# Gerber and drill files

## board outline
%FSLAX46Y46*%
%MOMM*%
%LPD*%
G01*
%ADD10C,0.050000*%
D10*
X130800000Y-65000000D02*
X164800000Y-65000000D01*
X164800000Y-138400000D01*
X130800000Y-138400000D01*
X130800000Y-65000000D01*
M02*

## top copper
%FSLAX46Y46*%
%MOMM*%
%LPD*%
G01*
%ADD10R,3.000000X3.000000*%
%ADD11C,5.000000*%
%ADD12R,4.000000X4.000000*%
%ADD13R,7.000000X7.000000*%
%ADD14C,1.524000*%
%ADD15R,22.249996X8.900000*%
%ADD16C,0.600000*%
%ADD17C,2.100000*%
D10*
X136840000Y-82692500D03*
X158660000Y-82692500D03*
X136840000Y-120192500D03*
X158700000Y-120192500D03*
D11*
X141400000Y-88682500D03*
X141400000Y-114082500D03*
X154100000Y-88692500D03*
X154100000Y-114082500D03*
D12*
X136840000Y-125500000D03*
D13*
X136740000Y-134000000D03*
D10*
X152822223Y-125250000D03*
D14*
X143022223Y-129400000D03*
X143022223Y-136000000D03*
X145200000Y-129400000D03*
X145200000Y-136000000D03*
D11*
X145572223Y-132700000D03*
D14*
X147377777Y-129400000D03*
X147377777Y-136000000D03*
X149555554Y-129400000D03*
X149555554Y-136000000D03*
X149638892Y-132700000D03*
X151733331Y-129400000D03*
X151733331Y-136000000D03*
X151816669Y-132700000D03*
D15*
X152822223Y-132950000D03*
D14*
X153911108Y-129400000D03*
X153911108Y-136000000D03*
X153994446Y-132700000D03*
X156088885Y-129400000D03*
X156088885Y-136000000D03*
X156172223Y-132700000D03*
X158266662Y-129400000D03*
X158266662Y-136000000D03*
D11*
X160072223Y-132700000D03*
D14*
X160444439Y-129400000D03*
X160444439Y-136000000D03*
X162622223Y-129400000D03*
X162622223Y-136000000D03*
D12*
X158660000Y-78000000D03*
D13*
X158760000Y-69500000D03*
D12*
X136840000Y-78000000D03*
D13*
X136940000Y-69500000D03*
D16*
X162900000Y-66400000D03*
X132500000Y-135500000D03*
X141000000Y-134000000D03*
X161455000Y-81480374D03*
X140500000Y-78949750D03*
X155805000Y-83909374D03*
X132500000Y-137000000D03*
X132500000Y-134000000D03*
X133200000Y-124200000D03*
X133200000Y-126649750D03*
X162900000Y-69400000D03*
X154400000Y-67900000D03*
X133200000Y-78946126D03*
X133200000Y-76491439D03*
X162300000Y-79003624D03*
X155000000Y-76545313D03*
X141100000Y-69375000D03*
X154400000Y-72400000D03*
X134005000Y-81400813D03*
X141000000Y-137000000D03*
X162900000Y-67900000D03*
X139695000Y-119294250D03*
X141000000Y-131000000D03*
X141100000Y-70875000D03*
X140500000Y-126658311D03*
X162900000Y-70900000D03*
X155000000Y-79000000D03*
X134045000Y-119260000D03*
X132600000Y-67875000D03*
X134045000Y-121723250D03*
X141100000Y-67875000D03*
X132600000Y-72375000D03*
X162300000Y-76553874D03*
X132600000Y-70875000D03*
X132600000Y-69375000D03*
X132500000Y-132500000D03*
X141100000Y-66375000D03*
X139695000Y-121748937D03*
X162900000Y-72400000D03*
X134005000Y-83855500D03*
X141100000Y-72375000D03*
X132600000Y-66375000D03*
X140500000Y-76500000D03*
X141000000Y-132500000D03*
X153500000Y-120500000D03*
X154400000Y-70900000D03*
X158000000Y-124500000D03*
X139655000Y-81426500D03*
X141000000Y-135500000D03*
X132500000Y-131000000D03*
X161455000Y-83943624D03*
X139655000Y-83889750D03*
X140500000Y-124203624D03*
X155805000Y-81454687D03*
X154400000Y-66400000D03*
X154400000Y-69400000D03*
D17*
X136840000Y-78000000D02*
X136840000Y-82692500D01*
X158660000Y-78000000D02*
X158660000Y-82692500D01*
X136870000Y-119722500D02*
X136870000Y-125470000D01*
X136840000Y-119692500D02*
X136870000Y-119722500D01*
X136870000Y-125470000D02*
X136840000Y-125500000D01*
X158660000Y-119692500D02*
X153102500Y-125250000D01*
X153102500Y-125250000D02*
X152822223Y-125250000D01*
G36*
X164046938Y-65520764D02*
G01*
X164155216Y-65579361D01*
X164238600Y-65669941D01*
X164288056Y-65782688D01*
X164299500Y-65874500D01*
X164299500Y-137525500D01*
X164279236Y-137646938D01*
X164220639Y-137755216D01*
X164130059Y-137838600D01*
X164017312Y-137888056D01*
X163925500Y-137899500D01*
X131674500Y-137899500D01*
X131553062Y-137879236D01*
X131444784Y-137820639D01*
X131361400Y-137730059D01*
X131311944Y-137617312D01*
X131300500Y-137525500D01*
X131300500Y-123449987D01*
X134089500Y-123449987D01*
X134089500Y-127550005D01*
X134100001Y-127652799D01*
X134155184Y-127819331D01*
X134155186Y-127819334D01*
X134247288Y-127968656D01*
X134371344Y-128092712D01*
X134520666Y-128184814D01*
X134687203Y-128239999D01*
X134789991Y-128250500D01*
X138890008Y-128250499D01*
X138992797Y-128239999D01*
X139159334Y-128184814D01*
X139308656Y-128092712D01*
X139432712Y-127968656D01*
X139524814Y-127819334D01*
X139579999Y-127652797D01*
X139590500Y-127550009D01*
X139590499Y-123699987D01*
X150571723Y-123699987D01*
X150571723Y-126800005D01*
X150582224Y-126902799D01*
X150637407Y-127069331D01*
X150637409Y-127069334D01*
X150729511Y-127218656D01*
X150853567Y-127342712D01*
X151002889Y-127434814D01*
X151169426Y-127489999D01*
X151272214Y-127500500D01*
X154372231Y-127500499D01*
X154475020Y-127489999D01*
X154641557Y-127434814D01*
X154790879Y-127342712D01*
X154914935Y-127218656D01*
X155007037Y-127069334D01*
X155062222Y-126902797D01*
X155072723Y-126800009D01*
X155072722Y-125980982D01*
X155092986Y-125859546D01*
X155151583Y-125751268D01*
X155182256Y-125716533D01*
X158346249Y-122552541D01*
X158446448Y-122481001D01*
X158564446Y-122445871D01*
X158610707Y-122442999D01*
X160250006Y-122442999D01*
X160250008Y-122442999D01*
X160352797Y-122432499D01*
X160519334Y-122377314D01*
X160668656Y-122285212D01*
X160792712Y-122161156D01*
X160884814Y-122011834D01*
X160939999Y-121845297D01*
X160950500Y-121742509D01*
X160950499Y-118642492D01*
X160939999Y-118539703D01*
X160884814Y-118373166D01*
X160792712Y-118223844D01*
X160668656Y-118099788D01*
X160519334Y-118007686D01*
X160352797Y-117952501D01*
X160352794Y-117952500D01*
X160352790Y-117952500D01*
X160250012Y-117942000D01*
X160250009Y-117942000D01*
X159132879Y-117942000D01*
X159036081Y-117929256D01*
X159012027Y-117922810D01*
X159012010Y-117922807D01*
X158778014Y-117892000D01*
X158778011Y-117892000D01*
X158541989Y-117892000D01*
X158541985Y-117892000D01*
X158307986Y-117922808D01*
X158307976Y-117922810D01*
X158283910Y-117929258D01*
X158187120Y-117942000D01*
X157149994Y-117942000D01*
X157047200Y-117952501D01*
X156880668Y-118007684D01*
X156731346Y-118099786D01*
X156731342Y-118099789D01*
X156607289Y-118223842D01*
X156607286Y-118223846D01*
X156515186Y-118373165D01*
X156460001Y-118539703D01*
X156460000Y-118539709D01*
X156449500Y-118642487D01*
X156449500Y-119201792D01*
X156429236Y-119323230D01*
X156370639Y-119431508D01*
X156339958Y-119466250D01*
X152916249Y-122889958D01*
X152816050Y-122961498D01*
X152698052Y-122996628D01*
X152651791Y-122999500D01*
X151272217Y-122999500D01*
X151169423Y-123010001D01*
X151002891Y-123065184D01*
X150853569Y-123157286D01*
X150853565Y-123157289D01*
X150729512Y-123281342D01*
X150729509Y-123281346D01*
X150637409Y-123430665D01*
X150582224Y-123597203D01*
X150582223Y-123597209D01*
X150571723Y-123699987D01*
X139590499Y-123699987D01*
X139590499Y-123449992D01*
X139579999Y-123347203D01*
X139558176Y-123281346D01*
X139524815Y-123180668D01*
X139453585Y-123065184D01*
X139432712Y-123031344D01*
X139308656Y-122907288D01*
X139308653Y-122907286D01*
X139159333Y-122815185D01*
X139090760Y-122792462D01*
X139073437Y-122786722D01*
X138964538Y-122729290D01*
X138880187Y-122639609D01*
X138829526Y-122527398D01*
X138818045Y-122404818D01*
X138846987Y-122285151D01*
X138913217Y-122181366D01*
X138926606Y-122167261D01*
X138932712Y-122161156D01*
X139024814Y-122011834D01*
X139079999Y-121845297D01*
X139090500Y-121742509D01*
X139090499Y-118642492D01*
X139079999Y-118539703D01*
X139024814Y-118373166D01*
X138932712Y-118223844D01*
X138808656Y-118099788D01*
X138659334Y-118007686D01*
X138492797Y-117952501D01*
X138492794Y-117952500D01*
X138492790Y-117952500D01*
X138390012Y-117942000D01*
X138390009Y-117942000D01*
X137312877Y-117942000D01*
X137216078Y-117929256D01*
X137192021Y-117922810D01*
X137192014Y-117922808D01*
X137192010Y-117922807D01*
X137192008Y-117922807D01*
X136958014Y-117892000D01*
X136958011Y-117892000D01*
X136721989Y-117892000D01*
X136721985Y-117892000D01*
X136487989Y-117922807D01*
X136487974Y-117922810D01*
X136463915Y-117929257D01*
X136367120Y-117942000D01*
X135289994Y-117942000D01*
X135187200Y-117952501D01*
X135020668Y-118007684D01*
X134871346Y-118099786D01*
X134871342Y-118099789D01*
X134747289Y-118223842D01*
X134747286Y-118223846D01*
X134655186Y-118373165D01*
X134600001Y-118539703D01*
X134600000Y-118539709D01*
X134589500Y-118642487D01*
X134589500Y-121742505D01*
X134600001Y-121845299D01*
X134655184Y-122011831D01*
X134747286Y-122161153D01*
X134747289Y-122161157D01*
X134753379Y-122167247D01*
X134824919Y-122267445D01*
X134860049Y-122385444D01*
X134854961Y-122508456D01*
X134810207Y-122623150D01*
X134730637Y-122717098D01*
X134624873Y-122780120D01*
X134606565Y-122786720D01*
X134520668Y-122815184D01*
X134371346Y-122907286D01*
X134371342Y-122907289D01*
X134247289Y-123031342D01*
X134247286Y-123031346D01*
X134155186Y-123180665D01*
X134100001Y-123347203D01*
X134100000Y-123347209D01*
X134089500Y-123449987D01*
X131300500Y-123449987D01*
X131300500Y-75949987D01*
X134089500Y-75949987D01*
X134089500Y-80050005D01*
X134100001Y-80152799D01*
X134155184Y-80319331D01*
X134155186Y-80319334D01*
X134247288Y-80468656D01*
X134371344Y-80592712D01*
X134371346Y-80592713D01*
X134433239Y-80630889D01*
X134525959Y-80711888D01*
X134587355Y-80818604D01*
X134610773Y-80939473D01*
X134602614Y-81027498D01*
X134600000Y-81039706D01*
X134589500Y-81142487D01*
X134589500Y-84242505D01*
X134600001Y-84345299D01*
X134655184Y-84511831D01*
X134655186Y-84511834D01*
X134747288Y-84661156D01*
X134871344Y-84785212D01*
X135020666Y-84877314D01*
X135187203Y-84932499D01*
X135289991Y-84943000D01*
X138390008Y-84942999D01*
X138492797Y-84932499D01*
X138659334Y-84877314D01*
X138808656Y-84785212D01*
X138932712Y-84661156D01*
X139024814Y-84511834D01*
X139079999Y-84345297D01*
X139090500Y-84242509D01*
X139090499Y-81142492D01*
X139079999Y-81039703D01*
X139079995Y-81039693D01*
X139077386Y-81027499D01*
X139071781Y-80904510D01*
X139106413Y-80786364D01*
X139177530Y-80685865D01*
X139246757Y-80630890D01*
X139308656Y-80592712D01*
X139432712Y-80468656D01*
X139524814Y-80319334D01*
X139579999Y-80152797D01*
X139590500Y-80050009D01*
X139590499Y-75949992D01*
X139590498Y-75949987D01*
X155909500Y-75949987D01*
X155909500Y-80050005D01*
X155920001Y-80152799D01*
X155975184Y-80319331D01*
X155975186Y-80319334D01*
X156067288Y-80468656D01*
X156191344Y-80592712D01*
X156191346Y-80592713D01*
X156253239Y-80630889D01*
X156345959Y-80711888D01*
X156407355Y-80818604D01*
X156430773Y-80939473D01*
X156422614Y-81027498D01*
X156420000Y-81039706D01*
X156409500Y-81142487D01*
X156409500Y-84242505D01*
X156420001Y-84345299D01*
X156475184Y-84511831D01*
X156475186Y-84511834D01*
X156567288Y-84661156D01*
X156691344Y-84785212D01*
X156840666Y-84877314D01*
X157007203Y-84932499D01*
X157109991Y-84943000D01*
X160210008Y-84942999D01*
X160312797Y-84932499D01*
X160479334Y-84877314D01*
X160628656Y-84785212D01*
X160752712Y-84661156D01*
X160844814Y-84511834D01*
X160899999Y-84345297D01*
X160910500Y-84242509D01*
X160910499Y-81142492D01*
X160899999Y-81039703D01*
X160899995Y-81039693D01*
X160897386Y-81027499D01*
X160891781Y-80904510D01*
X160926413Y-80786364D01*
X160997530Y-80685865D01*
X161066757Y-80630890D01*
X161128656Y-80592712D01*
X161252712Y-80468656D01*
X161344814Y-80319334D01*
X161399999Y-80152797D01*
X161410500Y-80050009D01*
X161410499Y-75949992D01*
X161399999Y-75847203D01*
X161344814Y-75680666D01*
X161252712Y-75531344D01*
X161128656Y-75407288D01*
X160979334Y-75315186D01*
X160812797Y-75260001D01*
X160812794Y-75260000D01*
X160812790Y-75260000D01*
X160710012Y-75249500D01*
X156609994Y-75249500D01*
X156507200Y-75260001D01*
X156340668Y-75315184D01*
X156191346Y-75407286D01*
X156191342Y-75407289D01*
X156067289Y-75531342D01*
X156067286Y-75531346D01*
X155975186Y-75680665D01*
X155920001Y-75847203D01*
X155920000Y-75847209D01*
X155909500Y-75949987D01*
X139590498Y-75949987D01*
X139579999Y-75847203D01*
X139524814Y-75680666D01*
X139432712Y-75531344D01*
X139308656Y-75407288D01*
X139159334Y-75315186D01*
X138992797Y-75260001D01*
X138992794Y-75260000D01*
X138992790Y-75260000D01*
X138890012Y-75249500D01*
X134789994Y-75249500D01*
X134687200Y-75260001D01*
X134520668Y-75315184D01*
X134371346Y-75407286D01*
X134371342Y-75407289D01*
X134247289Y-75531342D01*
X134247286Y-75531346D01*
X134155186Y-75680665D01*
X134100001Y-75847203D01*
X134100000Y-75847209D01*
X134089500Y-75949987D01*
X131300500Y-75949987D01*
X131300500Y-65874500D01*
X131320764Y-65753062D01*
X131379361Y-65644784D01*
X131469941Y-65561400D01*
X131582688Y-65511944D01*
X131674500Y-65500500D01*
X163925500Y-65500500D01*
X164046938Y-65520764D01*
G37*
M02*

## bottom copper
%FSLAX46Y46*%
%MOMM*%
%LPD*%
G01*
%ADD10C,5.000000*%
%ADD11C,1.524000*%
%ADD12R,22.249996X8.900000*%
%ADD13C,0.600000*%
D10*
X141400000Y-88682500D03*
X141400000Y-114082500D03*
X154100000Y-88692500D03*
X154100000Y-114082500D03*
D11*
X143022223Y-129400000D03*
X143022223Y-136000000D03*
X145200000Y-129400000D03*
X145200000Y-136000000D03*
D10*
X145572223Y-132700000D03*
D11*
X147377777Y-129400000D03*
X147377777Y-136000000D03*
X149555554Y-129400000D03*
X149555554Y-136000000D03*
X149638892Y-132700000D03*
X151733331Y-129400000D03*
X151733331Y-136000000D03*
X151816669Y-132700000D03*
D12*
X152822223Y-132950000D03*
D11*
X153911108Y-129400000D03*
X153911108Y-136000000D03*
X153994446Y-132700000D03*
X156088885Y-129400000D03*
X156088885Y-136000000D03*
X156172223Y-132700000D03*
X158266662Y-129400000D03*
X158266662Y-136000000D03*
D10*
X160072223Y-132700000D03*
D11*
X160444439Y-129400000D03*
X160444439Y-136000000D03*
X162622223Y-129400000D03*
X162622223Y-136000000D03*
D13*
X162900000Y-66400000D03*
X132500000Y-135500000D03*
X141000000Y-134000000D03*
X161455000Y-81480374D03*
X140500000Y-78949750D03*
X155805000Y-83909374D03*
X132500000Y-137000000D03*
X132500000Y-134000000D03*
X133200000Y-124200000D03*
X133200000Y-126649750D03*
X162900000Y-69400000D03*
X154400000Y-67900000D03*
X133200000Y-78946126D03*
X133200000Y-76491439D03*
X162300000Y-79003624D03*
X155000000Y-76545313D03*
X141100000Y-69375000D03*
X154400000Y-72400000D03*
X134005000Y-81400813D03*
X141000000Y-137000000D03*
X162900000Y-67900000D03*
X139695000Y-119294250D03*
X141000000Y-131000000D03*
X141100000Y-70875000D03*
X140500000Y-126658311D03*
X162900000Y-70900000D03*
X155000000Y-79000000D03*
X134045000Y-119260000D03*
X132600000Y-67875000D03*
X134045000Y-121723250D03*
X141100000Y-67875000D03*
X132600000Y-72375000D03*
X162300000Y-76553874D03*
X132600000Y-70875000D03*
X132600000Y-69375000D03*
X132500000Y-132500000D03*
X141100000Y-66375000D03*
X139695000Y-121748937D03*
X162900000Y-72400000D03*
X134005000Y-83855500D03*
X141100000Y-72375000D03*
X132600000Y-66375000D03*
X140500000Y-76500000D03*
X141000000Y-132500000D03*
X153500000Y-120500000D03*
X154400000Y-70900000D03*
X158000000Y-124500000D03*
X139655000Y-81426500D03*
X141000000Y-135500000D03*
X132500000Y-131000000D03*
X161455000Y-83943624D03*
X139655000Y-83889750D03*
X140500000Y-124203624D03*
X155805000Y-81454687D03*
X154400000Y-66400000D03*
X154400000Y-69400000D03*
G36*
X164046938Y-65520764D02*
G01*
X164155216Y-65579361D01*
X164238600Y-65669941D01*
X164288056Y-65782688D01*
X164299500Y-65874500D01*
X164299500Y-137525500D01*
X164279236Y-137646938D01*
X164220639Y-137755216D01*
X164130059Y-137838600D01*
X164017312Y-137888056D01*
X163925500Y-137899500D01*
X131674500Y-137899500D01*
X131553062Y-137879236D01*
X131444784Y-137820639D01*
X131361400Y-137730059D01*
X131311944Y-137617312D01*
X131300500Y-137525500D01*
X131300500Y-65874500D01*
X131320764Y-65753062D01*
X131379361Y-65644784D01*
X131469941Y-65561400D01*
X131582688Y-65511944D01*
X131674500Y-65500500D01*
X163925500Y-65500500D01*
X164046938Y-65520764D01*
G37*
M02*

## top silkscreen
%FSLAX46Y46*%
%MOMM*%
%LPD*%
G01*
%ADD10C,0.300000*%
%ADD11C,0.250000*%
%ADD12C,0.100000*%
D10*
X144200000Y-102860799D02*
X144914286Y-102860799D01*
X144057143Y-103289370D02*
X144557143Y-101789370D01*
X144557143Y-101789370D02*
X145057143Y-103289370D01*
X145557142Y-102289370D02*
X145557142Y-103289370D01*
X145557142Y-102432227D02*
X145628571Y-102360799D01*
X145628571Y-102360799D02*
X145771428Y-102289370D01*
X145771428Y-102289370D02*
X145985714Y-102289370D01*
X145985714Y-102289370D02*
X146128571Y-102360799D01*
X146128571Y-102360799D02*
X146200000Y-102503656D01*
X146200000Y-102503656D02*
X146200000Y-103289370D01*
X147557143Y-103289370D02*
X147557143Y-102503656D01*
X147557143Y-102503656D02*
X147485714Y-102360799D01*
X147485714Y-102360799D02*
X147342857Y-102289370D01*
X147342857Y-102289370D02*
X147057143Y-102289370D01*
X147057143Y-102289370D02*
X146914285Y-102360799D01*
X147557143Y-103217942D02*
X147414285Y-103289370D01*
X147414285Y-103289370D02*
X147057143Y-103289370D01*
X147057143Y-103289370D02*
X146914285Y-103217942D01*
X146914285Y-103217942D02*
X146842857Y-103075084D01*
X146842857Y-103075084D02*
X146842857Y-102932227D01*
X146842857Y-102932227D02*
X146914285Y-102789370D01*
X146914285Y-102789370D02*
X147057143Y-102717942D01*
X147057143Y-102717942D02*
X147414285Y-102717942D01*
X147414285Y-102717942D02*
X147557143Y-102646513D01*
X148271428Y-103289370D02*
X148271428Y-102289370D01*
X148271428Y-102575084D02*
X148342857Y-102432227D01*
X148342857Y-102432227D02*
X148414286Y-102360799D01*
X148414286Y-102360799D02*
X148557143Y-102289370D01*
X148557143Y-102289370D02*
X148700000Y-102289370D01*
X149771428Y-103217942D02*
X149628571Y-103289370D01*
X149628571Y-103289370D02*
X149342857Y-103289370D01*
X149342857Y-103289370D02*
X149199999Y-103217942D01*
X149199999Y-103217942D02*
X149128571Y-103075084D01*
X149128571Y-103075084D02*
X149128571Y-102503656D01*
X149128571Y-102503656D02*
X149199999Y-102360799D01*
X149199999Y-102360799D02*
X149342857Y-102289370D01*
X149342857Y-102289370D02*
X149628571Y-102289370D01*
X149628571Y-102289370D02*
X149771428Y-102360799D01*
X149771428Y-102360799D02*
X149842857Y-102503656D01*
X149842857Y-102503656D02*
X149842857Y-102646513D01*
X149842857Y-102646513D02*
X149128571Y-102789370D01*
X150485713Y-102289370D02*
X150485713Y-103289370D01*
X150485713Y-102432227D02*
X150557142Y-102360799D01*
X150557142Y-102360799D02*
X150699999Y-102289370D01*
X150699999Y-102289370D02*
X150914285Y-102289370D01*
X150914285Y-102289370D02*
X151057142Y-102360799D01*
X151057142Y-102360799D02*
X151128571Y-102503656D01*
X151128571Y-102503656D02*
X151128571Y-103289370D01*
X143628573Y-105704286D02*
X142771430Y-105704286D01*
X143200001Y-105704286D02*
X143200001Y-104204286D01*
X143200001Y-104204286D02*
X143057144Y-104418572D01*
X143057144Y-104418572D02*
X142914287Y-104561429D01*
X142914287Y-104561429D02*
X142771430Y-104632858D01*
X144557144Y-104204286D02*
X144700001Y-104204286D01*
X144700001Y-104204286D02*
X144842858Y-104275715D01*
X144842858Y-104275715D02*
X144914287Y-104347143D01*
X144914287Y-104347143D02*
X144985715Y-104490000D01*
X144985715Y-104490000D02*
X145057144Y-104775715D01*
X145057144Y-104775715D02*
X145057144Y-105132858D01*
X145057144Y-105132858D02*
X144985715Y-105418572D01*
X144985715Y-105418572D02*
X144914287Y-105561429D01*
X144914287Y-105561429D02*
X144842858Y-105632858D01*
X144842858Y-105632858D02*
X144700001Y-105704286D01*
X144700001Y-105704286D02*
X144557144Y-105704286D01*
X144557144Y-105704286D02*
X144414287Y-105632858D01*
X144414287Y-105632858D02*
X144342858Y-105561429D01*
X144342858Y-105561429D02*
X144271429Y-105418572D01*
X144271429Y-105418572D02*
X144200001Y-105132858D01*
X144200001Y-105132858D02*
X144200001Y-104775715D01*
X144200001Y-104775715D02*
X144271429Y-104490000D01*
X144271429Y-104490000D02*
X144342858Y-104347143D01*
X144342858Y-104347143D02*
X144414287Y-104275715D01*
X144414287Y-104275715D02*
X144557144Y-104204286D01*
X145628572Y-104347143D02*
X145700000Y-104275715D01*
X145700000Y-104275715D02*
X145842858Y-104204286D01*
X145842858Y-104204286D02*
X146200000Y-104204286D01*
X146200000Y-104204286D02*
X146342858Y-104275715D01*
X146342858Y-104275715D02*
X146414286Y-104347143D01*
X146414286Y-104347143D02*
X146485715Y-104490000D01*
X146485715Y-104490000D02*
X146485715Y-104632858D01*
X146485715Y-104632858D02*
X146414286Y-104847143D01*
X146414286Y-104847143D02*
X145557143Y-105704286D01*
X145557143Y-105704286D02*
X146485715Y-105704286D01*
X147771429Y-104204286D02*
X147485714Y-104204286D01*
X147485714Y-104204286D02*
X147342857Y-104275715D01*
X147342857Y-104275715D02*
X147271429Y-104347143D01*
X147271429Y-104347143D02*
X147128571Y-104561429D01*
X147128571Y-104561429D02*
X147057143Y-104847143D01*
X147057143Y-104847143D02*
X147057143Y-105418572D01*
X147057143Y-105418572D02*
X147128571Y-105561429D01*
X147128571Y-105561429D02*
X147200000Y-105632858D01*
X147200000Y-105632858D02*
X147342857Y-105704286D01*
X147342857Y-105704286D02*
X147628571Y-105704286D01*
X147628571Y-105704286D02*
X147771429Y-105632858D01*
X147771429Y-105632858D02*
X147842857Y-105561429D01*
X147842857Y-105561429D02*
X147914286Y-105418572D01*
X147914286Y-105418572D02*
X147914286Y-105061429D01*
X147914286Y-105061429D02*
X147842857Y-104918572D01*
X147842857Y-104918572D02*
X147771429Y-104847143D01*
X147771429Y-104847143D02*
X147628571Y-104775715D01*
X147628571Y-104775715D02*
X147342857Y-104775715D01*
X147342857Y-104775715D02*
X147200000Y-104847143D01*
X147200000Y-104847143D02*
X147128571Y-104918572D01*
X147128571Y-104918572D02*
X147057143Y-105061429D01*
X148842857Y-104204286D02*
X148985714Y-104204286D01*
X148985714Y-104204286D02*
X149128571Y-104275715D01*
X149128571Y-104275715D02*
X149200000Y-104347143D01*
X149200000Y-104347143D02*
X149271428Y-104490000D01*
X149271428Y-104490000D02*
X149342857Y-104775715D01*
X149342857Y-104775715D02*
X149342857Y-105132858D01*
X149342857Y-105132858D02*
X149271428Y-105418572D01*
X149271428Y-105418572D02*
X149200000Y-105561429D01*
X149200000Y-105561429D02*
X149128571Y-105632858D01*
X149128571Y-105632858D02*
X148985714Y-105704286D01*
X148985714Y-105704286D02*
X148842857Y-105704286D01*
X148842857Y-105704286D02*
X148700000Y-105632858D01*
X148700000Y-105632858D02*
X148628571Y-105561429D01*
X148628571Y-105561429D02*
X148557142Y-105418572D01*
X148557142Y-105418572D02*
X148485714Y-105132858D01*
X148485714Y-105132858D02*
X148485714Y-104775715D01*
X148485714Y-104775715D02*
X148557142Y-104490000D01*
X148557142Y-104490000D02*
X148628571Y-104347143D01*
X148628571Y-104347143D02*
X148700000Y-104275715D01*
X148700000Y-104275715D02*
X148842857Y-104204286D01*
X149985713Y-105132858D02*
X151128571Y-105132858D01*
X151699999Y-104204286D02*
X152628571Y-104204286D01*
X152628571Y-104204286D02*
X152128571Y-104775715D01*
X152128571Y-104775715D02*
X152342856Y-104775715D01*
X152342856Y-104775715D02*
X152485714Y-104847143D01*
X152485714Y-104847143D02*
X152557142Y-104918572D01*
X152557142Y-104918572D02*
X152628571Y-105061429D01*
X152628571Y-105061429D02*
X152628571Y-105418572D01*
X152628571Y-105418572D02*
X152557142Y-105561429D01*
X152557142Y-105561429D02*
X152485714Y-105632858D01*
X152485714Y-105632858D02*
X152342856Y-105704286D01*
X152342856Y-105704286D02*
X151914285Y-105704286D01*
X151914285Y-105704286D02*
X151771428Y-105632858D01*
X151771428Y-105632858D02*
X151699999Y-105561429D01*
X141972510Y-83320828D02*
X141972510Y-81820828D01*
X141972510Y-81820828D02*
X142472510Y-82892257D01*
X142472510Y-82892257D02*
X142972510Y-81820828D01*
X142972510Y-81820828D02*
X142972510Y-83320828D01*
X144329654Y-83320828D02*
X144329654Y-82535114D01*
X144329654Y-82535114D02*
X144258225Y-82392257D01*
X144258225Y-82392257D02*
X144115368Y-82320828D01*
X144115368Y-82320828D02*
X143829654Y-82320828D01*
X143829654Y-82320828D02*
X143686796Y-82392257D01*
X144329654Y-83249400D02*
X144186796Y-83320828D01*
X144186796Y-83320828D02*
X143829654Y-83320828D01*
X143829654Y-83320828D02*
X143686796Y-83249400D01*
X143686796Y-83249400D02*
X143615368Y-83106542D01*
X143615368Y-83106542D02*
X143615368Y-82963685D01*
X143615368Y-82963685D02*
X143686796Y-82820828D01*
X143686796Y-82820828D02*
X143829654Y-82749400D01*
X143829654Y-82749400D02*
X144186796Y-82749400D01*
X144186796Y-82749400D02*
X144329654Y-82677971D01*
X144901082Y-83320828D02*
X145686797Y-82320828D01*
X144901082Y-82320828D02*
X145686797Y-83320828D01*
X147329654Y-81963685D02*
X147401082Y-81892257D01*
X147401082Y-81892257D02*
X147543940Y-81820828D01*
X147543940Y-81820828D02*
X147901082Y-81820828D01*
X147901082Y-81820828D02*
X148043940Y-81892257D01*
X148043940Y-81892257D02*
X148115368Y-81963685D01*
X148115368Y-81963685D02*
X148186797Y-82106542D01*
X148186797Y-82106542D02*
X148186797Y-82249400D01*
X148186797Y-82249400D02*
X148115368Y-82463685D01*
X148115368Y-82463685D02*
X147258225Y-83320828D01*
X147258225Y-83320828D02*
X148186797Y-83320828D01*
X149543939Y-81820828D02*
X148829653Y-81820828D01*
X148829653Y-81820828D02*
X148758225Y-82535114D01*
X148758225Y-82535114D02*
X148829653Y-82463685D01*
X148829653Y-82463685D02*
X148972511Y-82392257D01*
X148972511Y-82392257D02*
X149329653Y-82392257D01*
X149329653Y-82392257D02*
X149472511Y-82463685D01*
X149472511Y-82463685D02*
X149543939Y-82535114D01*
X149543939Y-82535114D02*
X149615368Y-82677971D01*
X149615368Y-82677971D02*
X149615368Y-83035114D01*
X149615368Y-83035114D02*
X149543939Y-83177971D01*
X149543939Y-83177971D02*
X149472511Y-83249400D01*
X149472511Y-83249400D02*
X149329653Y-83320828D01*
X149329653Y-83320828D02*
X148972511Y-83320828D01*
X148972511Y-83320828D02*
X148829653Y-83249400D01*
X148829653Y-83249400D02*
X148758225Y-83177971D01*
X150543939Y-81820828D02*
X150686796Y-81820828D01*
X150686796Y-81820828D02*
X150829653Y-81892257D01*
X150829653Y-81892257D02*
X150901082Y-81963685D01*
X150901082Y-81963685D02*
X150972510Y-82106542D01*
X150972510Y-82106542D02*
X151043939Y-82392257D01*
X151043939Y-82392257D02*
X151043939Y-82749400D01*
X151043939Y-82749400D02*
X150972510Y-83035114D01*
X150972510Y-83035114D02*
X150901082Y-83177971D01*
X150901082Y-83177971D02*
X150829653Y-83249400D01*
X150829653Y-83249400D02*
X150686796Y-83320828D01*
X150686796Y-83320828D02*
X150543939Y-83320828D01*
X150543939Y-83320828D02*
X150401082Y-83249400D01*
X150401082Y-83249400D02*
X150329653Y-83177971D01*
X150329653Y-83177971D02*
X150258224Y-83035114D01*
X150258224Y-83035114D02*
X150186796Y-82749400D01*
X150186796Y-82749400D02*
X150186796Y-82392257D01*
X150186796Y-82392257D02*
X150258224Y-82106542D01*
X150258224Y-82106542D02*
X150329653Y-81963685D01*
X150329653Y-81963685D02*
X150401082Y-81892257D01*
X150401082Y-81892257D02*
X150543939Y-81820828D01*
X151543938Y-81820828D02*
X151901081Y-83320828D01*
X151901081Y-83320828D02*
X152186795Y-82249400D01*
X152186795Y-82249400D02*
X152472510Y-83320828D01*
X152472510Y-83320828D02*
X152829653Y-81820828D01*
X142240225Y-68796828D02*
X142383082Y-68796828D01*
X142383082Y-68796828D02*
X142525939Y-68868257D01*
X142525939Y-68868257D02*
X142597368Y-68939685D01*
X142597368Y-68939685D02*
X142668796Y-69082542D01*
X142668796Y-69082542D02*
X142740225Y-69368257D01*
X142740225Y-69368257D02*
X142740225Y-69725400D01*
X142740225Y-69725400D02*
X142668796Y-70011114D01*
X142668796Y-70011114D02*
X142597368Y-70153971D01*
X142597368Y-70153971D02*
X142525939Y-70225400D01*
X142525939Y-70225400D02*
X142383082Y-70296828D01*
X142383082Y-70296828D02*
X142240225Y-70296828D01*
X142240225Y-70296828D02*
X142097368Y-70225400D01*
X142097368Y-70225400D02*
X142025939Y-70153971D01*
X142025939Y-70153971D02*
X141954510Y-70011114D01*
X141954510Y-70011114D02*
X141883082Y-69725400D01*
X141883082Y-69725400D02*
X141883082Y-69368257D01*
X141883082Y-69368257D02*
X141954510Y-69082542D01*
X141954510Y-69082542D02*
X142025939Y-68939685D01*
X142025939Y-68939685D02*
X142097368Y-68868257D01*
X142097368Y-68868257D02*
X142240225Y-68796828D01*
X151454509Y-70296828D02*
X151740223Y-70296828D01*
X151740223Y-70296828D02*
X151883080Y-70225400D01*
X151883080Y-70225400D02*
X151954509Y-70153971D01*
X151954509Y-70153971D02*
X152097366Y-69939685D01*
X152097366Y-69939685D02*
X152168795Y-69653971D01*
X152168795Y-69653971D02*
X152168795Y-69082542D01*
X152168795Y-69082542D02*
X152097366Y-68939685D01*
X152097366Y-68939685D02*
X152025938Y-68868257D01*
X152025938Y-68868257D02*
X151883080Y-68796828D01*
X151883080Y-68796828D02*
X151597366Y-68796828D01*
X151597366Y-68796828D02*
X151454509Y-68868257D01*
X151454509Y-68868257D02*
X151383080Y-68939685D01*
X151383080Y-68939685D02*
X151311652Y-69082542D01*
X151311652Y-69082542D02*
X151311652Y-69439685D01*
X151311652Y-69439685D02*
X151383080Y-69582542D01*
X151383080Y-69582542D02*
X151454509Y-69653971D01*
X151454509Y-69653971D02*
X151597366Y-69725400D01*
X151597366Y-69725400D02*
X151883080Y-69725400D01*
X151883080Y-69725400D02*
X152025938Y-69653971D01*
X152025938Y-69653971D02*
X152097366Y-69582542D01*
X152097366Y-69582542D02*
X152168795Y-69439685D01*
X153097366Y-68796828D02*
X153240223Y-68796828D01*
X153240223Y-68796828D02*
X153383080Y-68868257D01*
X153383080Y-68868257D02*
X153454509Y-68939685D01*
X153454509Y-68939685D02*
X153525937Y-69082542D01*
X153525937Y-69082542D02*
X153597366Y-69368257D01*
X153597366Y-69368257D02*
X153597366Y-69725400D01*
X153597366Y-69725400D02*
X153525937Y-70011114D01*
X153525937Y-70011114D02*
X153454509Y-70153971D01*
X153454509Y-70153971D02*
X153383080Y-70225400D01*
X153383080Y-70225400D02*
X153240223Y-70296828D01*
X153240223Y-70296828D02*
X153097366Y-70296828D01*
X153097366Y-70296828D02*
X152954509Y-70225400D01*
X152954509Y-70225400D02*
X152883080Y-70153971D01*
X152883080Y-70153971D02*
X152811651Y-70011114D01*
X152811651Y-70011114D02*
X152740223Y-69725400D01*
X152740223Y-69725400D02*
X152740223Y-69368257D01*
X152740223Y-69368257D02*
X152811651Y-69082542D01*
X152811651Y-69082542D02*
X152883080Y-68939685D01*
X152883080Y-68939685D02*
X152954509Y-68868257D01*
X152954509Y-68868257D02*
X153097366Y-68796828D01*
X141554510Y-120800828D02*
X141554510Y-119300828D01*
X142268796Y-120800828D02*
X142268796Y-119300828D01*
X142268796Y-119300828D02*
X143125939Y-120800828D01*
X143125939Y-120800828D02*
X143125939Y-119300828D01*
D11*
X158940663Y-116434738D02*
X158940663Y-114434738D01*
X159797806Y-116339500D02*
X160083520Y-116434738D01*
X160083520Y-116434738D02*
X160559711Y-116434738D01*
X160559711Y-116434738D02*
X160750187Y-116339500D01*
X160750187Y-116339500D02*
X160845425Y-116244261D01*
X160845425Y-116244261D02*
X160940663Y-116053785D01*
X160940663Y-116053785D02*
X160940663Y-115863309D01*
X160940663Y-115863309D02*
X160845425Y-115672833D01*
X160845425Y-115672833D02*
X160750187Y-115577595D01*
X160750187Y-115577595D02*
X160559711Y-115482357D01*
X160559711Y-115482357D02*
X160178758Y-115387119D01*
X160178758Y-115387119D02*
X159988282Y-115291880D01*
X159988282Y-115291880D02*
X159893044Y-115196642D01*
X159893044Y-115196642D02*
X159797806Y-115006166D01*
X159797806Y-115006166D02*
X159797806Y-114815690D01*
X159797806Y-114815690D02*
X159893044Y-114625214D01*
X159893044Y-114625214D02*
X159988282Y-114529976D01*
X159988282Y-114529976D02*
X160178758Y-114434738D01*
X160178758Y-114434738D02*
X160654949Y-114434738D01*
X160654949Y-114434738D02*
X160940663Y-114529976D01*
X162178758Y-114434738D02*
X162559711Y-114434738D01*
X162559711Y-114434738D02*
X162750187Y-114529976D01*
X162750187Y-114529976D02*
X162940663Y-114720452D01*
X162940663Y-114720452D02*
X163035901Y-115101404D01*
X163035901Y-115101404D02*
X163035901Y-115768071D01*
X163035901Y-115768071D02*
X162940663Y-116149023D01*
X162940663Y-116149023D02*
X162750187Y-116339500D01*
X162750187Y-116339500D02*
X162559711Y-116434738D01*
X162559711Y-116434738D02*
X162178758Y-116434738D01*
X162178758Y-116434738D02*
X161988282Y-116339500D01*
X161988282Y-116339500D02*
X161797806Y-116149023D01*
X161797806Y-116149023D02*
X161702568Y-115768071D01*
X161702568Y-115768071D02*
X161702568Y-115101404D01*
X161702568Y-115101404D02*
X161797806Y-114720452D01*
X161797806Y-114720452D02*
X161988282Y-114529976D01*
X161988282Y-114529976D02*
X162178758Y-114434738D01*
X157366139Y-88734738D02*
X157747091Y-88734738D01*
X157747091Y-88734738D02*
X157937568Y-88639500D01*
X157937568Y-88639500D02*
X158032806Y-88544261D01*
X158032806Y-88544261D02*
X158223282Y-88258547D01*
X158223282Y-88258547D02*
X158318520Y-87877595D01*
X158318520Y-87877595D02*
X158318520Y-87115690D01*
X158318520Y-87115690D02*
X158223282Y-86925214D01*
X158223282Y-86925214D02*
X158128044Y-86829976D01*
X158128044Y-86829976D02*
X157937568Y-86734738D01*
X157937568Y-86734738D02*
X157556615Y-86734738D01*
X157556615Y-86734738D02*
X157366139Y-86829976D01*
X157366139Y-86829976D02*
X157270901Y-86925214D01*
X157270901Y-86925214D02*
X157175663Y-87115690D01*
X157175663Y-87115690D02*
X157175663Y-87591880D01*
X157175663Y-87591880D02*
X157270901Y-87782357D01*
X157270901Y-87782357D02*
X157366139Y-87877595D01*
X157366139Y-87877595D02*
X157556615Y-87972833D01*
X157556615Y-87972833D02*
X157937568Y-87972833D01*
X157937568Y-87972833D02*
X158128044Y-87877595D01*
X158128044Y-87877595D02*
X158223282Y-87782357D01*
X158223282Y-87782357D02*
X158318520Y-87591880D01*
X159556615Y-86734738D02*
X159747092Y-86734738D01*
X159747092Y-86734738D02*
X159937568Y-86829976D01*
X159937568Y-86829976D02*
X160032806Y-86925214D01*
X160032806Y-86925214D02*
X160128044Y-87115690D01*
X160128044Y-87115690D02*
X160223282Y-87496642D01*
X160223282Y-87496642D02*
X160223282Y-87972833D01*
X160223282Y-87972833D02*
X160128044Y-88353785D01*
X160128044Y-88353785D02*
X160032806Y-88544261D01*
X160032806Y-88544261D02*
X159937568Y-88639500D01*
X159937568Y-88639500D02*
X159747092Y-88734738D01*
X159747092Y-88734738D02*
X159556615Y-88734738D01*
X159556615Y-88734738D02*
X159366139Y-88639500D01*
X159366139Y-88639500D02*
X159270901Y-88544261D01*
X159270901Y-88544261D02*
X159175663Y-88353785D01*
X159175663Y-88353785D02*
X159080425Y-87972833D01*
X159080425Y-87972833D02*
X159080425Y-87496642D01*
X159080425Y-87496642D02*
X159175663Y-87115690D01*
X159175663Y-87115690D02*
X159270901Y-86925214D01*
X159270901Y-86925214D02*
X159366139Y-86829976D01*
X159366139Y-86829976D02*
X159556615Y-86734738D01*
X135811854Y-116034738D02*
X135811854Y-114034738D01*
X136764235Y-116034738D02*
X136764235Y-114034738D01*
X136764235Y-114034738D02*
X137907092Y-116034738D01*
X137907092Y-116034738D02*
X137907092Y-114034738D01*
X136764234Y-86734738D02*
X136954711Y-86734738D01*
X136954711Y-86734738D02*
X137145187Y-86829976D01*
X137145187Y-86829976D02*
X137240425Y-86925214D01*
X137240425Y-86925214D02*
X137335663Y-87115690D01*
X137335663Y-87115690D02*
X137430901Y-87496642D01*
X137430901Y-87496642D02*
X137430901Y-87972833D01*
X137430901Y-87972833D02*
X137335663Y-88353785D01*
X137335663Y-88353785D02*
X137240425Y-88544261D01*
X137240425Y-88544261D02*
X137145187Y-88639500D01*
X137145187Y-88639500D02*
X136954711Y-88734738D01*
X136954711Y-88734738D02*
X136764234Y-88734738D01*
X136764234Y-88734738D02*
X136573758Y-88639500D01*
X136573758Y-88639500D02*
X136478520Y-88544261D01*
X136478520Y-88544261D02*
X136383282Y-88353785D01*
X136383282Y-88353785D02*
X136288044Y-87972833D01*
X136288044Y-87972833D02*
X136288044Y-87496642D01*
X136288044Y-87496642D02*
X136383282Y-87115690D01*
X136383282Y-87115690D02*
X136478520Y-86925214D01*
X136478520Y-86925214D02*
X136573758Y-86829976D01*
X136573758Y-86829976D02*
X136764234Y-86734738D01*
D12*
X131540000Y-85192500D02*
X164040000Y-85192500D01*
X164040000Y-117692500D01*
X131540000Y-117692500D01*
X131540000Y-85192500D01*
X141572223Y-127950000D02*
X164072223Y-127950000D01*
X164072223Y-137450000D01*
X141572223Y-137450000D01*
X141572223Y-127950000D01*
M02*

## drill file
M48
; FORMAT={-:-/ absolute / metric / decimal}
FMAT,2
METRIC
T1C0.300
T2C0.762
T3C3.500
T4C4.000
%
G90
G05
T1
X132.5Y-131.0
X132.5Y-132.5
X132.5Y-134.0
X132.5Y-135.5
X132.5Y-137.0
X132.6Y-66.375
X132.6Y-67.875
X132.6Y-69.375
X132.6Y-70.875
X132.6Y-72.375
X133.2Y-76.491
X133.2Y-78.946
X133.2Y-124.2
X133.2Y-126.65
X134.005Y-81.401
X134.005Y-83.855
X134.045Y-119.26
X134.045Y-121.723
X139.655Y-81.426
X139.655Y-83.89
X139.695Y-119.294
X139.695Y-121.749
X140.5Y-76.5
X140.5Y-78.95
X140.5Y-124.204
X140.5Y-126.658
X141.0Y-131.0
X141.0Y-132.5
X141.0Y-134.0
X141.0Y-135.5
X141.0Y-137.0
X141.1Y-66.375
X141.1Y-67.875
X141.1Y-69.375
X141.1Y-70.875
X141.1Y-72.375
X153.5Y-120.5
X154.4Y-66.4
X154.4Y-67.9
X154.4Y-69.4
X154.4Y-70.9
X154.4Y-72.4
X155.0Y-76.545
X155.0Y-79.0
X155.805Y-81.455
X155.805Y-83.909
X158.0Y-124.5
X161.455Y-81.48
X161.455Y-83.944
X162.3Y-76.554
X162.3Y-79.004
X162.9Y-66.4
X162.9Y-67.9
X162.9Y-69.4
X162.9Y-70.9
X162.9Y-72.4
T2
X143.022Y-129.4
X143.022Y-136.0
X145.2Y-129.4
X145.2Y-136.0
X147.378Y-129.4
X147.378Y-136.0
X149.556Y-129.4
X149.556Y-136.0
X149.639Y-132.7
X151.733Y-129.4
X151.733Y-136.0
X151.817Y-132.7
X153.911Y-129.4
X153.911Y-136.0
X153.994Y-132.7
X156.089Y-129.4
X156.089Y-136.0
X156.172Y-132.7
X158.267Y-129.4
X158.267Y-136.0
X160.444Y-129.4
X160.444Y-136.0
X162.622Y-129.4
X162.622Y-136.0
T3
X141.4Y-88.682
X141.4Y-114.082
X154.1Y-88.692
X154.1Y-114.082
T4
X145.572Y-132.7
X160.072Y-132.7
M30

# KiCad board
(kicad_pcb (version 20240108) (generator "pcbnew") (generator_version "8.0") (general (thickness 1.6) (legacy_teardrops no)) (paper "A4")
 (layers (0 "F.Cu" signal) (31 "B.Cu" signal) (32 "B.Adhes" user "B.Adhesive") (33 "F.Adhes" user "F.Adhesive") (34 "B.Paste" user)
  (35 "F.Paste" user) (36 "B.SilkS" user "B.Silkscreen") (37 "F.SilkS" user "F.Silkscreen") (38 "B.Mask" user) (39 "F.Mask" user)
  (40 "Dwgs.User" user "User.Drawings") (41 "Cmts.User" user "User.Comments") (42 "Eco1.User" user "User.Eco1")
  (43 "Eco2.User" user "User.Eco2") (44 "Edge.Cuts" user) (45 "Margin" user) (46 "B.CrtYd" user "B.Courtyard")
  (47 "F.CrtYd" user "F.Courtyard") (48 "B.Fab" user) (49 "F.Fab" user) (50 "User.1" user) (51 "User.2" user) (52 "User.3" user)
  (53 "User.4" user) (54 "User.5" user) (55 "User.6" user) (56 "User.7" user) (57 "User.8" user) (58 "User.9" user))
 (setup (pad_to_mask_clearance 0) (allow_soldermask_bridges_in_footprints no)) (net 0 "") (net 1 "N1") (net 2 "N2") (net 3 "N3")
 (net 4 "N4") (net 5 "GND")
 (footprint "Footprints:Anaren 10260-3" (layer "F.Cu") (at 148.7 101.6925)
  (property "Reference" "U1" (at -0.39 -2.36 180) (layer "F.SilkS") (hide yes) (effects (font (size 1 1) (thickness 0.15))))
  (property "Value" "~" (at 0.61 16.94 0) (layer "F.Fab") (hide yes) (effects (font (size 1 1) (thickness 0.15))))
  (fp_rect (start -17.16 -16.5) (end 15.34 16) (stroke (width 0.1) (type default)) (fill none) (layer "F.SilkS"))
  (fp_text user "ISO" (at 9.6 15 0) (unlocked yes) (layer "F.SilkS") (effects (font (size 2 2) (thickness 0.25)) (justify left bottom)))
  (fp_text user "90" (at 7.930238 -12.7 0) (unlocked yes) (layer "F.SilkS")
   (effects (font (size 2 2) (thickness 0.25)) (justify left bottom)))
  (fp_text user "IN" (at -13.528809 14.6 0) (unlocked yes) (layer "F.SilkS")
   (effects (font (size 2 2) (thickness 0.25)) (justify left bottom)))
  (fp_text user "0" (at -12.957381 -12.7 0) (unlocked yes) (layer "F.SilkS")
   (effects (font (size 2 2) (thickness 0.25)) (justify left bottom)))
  (pad "1" smd rect (at -11.86 -19 270) (size 3 3) (layers "F.Cu" "F.Paste" "F.Mask") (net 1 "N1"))
  (pad "2" smd rect (at 9.96 -19 270) (size 3 3) (layers "F.Cu" "F.Paste" "F.Mask") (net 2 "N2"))
  (pad "3" smd rect (at -11.86 18.5 270) (size 3 3) (layers "F.Cu" "F.Paste" "F.Mask") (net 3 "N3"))
  (pad "4" smd rect (at 10 18.5 270) (size 3 3) (layers "F.Cu" "F.Paste" "F.Mask") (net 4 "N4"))
  (pad "5" thru_hole circle (at -7.3 -13.01) (size 5 5) (drill 3.5) (layers "*.Cu" "*.Mask") (remove_unused_layers no) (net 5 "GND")
   (zone_connect 2))
  (pad "5" thru_hole circle (at -7.3 12.39) (size 5 5) (drill 3.5) (layers "*.Cu" "*.Mask") (remove_unused_layers no) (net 5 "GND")
   (zone_connect 2))
  (pad "5" thru_hole circle (at 5.4 -13) (size 5 5) (drill 3.5) (layers "*.Cu" "*.Mask") (remove_unused_layers no) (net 5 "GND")
   (zone_connect 2))
  (pad "5" thru_hole circle (at 5.4 12.39) (size 5 5) (drill 3.5) (layers "*.Cu" "*.Mask") (remove_unused_layers no) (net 5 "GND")
   (zone_connect 2)))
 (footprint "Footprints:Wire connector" (layer "F.Cu") (at 136.84 129.5 -90)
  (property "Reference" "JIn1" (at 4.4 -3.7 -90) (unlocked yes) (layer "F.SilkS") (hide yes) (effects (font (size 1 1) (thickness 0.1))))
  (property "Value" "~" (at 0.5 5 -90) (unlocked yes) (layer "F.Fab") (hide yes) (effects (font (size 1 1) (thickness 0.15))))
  (pad "1" smd rect (at -4 0 180) (size 4 4) (layers "F.Cu" "F.Paste" "F.Mask") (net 3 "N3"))
  (pad "2" smd rect (at 4.5 0.1 180) (size 7 7) (layers "F.Cu" "F.Paste" "F.Mask") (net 5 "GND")))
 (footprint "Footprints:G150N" (layer "F.Cu") (at 152.822223 133.25)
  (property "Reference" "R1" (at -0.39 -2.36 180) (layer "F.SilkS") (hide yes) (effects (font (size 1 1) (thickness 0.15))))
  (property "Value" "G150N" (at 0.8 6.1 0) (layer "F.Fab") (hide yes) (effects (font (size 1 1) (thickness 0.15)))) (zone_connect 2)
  (fp_rect (start -11.25 -5.3) (end 11.25 4.2) (stroke (width 0.1) (type default)) (fill none) (layer "F.SilkS"))
  (pad "1" smd rect (at 0 -8 270) (size 3 3) (layers "F.Cu" "F.Paste" "F.Mask") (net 4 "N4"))
  (pad "2" thru_hole circle (at -9.8 -3.85) (size 1.524 1.524) (drill 0.762) (layers "*.Cu" "*.Mask") (remove_unused_layers no)
   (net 5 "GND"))
  (pad "2" thru_hole circle (at -9.8 2.75) (size 1.524 1.524) (drill 0.762) (layers "*.Cu" "*.Mask") (remove_unused_layers no) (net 5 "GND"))
  (pad "2" thru_hole circle (at -7.622223 -3.85) (size 1.524 1.524) (drill 0.762) (layers "*.Cu" "*.Mask") (remove_unused_layers no)
   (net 5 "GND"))
  (pad "2" thru_hole circle (at -7.622223 2.75) (size 1.524 1.524) (drill 0.762) (layers "*.Cu" "*.Mask") (remove_unused_layers no)
   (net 5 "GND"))
  (pad "2" thru_hole circle (at -7.25 -0.55 270) (size 5 5) (drill 4) (layers "*.Cu" "*.Mask") (remove_unused_layers no) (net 5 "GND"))
  (pad "2" thru_hole circle (at -5.444446 -3.85) (size 1.524 1.524) (drill 0.762) (layers "*.Cu" "*.Mask") (remove_unused_layers no)
   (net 5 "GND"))
  (pad "2" thru_hole circle (at -5.444446 2.75) (size 1.524 1.524) (drill 0.762) (layers "*.Cu" "*.Mask") (remove_unused_layers no)
   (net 5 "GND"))
  (pad "2" thru_hole circle (at -3.266669 -3.85) (size 1.524 1.524) (drill 0.762) (layers "*.Cu" "*.Mask") (remove_unused_layers no)
   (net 5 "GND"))
  (pad "2" thru_hole circle (at -3.266669 2.75) (size 1.524 1.524) (drill 0.762) (layers "*.Cu" "*.Mask") (remove_unused_layers no)
   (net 5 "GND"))
  (pad "2" thru_hole circle (at -3.183331 -0.55) (size 1.524 1.524) (drill 0.762) (layers "*.Cu" "*.Mask") (remove_unused_layers no)
   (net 5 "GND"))
  (pad "2" thru_hole circle (at -1.088892 -3.85) (size 1.524 1.524) (drill 0.762) (layers "*.Cu" "*.Mask") (remove_unused_layers no)
   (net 5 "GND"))
  (pad "2" thru_hole circle (at -1.088892 2.75) (size 1.524 1.524) (drill 0.762) (layers "*.Cu" "*.Mask") (remove_unused_layers no)
   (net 5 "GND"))
  (pad "2" thru_hole circle (at -1.005554 -0.55) (size 1.524 1.524) (drill 0.762) (layers "*.Cu" "*.Mask") (remove_unused_layers no)
   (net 5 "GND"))
  (pad "2" smd rect (at 0 -0.3 270) (size 8.9 22.249996) (layers "F.Cu" "F.Mask") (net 5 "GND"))
  (pad "2" smd rect (at 0 -0.3 270) (size 8.9 22.249996) (layers "B.Cu" "B.Mask") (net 5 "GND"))
  (pad "2" thru_hole circle (at 1.088885 -3.85) (size 1.524 1.524) (drill 0.762) (layers "*.Cu" "*.Mask") (remove_unused_layers no)
   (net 5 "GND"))
  (pad "2" thru_hole circle (at 1.088885 2.75) (size 1.524 1.524) (drill 0.762) (layers "*.Cu" "*.Mask") (remove_unused_layers no)
   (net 5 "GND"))
  (pad "2" thru_hole circle (at 1.172223 -0.55) (size 1.524 1.524) (drill 0.762) (layers "*.Cu" "*.Mask") (remove_unused_layers no)
   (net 5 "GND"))
  (pad "2" thru_hole circle (at 3.266662 -3.85) (size 1.524 1.524) (drill 0.762) (layers "*.Cu" "*.Mask") (remove_unused_layers no)
   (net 5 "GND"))
  (pad "2" thru_hole circle (at 3.266662 2.75) (size 1.524 1.524) (drill 0.762) (layers "*.Cu" "*.Mask") (remove_unused_layers no)
   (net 5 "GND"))
  (pad "2" thru_hole circle (at 3.35 -0.55) (size 1.524 1.524) (drill 0.762) (layers "*.Cu" "*.Mask") (remove_unused_layers no)
   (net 5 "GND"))
  (pad "2" thru_hole circle (at 5.444439 -3.85) (size 1.524 1.524) (drill 0.762) (layers "*.Cu" "*.Mask") (remove_unused_layers no)
   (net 5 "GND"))
  (pad "2" thru_hole circle (at 5.444439 2.75) (size 1.524 1.524) (drill 0.762) (layers "*.Cu" "*.Mask") (remove_unused_layers no)
   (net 5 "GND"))
  (pad "2" thru_hole circle (at 7.25 -0.55 270) (size 5 5) (drill 4) (layers "*.Cu" "*.Mask") (remove_unused_layers no) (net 5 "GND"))
  (pad "2" thru_hole circle (at 7.622216 -3.85) (size 1.524 1.524) (drill 0.762) (layers "*.Cu" "*.Mask") (remove_unused_layers no)
   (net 5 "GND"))
  (pad "2" thru_hole circle (at 7.622216 2.75) (size 1.524 1.524) (drill 0.762) (layers "*.Cu" "*.Mask") (remove_unused_layers no)
   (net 5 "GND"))
  (pad "2" thru_hole circle (at 9.8 -3.85) (size 1.524 1.524) (drill 0.762) (layers "*.Cu" "*.Mask") (remove_unused_layers no) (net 5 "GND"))
  (pad "2" thru_hole circle (at 9.8 2.75) (size 1.524 1.524) (drill 0.762) (layers "*.Cu" "*.Mask") (remove_unused_layers no) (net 5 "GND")))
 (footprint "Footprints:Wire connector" (layer "F.Cu") (at 158.66 74 90)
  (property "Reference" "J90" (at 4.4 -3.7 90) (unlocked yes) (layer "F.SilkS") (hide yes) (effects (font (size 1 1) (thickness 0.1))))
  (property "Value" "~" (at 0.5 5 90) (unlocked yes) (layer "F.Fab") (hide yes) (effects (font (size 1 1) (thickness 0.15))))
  (pad "1" smd rect (at -4 0) (size 4 4) (layers "F.Cu" "F.Paste" "F.Mask") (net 2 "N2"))
  (pad "2" smd rect (at 4.5 0.1) (size 7 7) (layers "F.Cu" "F.Paste" "F.Mask") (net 5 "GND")))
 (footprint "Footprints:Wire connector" (layer "F.Cu") (at 136.84 74 90)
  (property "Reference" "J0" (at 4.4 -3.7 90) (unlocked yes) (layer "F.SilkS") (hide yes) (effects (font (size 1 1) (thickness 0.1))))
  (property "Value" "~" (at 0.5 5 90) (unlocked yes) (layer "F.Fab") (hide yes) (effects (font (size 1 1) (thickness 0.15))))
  (pad "1" smd rect (at -4 0) (size 4 4) (layers "F.Cu" "F.Paste" "F.Mask") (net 1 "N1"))
  (pad "2" smd rect (at 4.5 0.1) (size 7 7) (layers "F.Cu" "F.Paste" "F.Mask") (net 5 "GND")))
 (gr_rect (start 130.8 65) (end 164.8 138.4) (stroke (width 0.05) (type default)) (fill none) (layer "Edge.Cuts"))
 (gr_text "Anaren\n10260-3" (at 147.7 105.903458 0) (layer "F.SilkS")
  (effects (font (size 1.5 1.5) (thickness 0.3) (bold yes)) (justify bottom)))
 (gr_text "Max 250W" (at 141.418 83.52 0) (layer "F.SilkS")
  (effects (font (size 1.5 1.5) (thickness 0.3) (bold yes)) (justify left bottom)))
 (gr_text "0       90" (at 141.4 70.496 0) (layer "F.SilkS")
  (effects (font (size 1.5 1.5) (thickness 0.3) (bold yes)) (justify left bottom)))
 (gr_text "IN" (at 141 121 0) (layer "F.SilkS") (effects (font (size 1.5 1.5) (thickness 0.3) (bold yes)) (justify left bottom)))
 (via (at 162.9 66.4) (size 0.6) (drill 0.3) (layers "F.Cu" "B.Cu") (free yes) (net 5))
 (via (at 132.5 135.5) (size 0.6) (drill 0.3) (layers "F.Cu" "B.Cu") (free yes) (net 5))
 (via (at 141 134) (size 0.6) (drill 0.3) (layers "F.Cu" "B.Cu") (free yes) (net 5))
 (via (at 161.455 81.480374) (size 0.6) (drill 0.3) (layers "F.Cu" "B.Cu") (free yes) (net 5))
 (via (at 140.5 78.94975) (size 0.6) (drill 0.3) (layers "F.Cu" "B.Cu") (free yes) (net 5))
 (via (at 155.805 83.909374) (size 0.6) (drill 0.3) (layers "F.Cu" "B.Cu") (free yes) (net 5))
 (via (at 132.5 137) (size 0.6) (drill 0.3) (layers "F.Cu" "B.Cu") (free yes) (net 5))
 (via (at 132.5 134) (size 0.6) (drill 0.3) (layers "F.Cu" "B.Cu") (free yes) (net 5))
 (via (at 133.2 124.2) (size 0.6) (drill 0.3) (layers "F.Cu" "B.Cu") (free yes) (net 5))
 (via (at 133.2 126.64975) (size 0.6) (drill 0.3) (layers "F.Cu" "B.Cu") (free yes) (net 5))
 (via (at 162.9 69.4) (size 0.6) (drill 0.3) (layers "F.Cu" "B.Cu") (free yes) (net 5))
 (via (at 154.4 67.9) (size 0.6) (drill 0.3) (layers "F.Cu" "B.Cu") (free yes) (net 5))
 (via (at 133.2 78.946126) (size 0.6) (drill 0.3) (layers "F.Cu" "B.Cu") (free yes) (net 5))
 (via (at 133.2 76.491439) (size 0.6) (drill 0.3) (layers "F.Cu" "B.Cu") (free yes) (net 5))
 (via (at 162.3 79.003624) (size 0.6) (drill 0.3) (layers "F.Cu" "B.Cu") (free yes) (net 5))
 (via (at 155 76.545313) (size 0.6) (drill 0.3) (layers "F.Cu" "B.Cu") (free yes) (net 5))
 (via (at 141.1 69.375) (size 0.6) (drill 0.3) (layers "F.Cu" "B.Cu") (free yes) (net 5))
 (via (at 154.4 72.4) (size 0.6) (drill 0.3) (layers "F.Cu" "B.Cu") (free yes) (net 5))
 (via (at 134.005 81.400813) (size 0.6) (drill 0.3) (layers "F.Cu" "B.Cu") (free yes) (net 5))
 (via (at 141 137) (size 0.6) (drill 0.3) (layers "F.Cu" "B.Cu") (free yes) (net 5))
 (via (at 162.9 67.9) (size 0.6) (drill 0.3) (layers "F.Cu" "B.Cu") (free yes) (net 5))
 (via (at 139.695 119.29425) (size 0.6) (drill 0.3) (layers "F.Cu" "B.Cu") (free yes) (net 5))
 (via (at 141 131) (size 0.6) (drill 0.3) (layers "F.Cu" "B.Cu") (free yes) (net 5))
 (via (at 141.1 70.875) (size 0.6) (drill 0.3) (layers "F.Cu" "B.Cu") (free yes) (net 5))
 (via (at 140.5 126.658311) (size 0.6) (drill 0.3) (layers "F.Cu" "B.Cu") (free yes) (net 5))
 (via (at 162.9 70.9) (size 0.6) (drill 0.3) (layers "F.Cu" "B.Cu") (free yes) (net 5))
 (via (at 155 79) (size 0.6) (drill 0.3) (layers "F.Cu" "B.Cu") (free yes) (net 5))
 (via (at 134.045 119.26) (size 0.6) (drill 0.3) (layers "F.Cu" "B.Cu") (free yes) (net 5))
 (via (at 132.6 67.875) (size 0.6) (drill 0.3) (layers "F.Cu" "B.Cu") (free yes) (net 5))
 (via (at 134.045 121.72325) (size 0.6) (drill 0.3) (layers "F.Cu" "B.Cu") (free yes) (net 5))
 (via (at 141.1 67.875) (size 0.6) (drill 0.3) (layers "F.Cu" "B.Cu") (free yes) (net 5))
 (via (at 132.6 72.375) (size 0.6) (drill 0.3) (layers "F.Cu" "B.Cu") (free yes) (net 5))
 (via (at 162.3 76.553874) (size 0.6) (drill 0.3) (layers "F.Cu" "B.Cu") (free yes) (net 5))
 (via (at 132.6 70.875) (size 0.6) (drill 0.3) (layers "F.Cu" "B.Cu") (free yes) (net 5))
 (via (at 132.6 69.375) (size 0.6) (drill 0.3) (layers "F.Cu" "B.Cu") (free yes) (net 5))
 (via (at 132.5 132.5) (size 0.6) (drill 0.3) (layers "F.Cu" "B.Cu") (free yes) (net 5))
 (via (at 141.1 66.375) (size 0.6) (drill 0.3) (layers "F.Cu" "B.Cu") (free yes) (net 5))
 (via (at 139.695 121.748937) (size 0.6) (drill 0.3) (layers "F.Cu" "B.Cu") (free yes) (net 5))
 (via (at 162.9 72.4) (size 0.6) (drill 0.3) (layers "F.Cu" "B.Cu") (free yes) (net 5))
 (via (at 134.005 83.8555) (size 0.6) (drill 0.3) (layers "F.Cu" "B.Cu") (free yes) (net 5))
 (via (at 141.1 72.375) (size 0.6) (drill 0.3) (layers "F.Cu" "B.Cu") (free yes) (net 5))
 (via (at 132.6 66.375) (size 0.6) (drill 0.3) (layers "F.Cu" "B.Cu") (free yes) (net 5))
 (via (at 140.5 76.5) (size 0.6) (drill 0.3) (layers "F.Cu" "B.Cu") (free yes) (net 5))
 (via (at 141 132.5) (size 0.6) (drill 0.3) (layers "F.Cu" "B.Cu") (free yes) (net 5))
 (via (at 153.5 120.5) (size 0.6) (drill 0.3) (layers "F.Cu" "B.Cu") (free yes) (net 5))
 (via (at 154.4 70.9) (size 0.6) (drill 0.3) (layers "F.Cu" "B.Cu") (free yes) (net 5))
 (via (at 158 124.5) (size 0.6) (drill 0.3) (layers "F.Cu" "B.Cu") (free yes) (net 5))
 (via (at 139.655 81.4265) (size 0.6) (drill 0.3) (layers "F.Cu" "B.Cu") (free yes) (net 5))
 (via (at 141 135.5) (size 0.6) (drill 0.3) (layers "F.Cu" "B.Cu") (free yes) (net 5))
 (via (at 132.5 131) (size 0.6) (drill 0.3) (layers "F.Cu" "B.Cu") (free yes) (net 5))
 (via (at 161.455 83.943624) (size 0.6) (drill 0.3) (layers "F.Cu" "B.Cu") (free yes) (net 5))
 (via (at 139.655 83.88975) (size 0.6) (drill 0.3) (layers "F.Cu" "B.Cu") (free yes) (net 5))
 (via (at 140.5 124.203624) (size 0.6) (drill 0.3) (layers "F.Cu" "B.Cu") (free yes) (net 5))
 (via (at 155.805 81.454687) (size 0.6) (drill 0.3) (layers "F.Cu" "B.Cu") (free yes) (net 5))
 (via (at 154.4 66.4) (size 0.6) (drill 0.3) (layers "F.Cu" "B.Cu") (free yes) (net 5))
 (via (at 154.4 69.4) (size 0.6) (drill 0.3) (layers "F.Cu" "B.Cu") (free yes) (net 5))
 (segment (start 136.84 78) (end 136.84 82.6925) (width 2.1) (layer "F.Cu") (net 1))
 (segment (start 158.66 78) (end 158.66 82.6925) (width 2.1) (layer "F.Cu") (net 2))
 (segment (start 136.87 119.7225) (end 136.87 125.47) (width 2.1) (layer "F.Cu") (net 3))
 (segment (start 136.84 119.6925) (end 136.87 119.7225) (width 2.1) (layer "F.Cu") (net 3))
 (segment (start 136.87 125.47) (end 136.84 125.5) (width 2.1) (layer "F.Cu") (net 3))
 (segment (start 158.66 119.6925) (end 153.1025 125.25) (width 2.1) (layer "F.Cu") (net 4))
 (segment (start 153.1025 125.25) (end 152.822223 125.25) (width 2.1) (layer "F.Cu") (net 4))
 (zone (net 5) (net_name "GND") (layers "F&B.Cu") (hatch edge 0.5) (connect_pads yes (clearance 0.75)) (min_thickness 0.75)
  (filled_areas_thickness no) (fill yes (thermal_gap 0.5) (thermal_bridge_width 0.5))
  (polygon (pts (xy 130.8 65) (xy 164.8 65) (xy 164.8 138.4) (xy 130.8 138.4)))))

